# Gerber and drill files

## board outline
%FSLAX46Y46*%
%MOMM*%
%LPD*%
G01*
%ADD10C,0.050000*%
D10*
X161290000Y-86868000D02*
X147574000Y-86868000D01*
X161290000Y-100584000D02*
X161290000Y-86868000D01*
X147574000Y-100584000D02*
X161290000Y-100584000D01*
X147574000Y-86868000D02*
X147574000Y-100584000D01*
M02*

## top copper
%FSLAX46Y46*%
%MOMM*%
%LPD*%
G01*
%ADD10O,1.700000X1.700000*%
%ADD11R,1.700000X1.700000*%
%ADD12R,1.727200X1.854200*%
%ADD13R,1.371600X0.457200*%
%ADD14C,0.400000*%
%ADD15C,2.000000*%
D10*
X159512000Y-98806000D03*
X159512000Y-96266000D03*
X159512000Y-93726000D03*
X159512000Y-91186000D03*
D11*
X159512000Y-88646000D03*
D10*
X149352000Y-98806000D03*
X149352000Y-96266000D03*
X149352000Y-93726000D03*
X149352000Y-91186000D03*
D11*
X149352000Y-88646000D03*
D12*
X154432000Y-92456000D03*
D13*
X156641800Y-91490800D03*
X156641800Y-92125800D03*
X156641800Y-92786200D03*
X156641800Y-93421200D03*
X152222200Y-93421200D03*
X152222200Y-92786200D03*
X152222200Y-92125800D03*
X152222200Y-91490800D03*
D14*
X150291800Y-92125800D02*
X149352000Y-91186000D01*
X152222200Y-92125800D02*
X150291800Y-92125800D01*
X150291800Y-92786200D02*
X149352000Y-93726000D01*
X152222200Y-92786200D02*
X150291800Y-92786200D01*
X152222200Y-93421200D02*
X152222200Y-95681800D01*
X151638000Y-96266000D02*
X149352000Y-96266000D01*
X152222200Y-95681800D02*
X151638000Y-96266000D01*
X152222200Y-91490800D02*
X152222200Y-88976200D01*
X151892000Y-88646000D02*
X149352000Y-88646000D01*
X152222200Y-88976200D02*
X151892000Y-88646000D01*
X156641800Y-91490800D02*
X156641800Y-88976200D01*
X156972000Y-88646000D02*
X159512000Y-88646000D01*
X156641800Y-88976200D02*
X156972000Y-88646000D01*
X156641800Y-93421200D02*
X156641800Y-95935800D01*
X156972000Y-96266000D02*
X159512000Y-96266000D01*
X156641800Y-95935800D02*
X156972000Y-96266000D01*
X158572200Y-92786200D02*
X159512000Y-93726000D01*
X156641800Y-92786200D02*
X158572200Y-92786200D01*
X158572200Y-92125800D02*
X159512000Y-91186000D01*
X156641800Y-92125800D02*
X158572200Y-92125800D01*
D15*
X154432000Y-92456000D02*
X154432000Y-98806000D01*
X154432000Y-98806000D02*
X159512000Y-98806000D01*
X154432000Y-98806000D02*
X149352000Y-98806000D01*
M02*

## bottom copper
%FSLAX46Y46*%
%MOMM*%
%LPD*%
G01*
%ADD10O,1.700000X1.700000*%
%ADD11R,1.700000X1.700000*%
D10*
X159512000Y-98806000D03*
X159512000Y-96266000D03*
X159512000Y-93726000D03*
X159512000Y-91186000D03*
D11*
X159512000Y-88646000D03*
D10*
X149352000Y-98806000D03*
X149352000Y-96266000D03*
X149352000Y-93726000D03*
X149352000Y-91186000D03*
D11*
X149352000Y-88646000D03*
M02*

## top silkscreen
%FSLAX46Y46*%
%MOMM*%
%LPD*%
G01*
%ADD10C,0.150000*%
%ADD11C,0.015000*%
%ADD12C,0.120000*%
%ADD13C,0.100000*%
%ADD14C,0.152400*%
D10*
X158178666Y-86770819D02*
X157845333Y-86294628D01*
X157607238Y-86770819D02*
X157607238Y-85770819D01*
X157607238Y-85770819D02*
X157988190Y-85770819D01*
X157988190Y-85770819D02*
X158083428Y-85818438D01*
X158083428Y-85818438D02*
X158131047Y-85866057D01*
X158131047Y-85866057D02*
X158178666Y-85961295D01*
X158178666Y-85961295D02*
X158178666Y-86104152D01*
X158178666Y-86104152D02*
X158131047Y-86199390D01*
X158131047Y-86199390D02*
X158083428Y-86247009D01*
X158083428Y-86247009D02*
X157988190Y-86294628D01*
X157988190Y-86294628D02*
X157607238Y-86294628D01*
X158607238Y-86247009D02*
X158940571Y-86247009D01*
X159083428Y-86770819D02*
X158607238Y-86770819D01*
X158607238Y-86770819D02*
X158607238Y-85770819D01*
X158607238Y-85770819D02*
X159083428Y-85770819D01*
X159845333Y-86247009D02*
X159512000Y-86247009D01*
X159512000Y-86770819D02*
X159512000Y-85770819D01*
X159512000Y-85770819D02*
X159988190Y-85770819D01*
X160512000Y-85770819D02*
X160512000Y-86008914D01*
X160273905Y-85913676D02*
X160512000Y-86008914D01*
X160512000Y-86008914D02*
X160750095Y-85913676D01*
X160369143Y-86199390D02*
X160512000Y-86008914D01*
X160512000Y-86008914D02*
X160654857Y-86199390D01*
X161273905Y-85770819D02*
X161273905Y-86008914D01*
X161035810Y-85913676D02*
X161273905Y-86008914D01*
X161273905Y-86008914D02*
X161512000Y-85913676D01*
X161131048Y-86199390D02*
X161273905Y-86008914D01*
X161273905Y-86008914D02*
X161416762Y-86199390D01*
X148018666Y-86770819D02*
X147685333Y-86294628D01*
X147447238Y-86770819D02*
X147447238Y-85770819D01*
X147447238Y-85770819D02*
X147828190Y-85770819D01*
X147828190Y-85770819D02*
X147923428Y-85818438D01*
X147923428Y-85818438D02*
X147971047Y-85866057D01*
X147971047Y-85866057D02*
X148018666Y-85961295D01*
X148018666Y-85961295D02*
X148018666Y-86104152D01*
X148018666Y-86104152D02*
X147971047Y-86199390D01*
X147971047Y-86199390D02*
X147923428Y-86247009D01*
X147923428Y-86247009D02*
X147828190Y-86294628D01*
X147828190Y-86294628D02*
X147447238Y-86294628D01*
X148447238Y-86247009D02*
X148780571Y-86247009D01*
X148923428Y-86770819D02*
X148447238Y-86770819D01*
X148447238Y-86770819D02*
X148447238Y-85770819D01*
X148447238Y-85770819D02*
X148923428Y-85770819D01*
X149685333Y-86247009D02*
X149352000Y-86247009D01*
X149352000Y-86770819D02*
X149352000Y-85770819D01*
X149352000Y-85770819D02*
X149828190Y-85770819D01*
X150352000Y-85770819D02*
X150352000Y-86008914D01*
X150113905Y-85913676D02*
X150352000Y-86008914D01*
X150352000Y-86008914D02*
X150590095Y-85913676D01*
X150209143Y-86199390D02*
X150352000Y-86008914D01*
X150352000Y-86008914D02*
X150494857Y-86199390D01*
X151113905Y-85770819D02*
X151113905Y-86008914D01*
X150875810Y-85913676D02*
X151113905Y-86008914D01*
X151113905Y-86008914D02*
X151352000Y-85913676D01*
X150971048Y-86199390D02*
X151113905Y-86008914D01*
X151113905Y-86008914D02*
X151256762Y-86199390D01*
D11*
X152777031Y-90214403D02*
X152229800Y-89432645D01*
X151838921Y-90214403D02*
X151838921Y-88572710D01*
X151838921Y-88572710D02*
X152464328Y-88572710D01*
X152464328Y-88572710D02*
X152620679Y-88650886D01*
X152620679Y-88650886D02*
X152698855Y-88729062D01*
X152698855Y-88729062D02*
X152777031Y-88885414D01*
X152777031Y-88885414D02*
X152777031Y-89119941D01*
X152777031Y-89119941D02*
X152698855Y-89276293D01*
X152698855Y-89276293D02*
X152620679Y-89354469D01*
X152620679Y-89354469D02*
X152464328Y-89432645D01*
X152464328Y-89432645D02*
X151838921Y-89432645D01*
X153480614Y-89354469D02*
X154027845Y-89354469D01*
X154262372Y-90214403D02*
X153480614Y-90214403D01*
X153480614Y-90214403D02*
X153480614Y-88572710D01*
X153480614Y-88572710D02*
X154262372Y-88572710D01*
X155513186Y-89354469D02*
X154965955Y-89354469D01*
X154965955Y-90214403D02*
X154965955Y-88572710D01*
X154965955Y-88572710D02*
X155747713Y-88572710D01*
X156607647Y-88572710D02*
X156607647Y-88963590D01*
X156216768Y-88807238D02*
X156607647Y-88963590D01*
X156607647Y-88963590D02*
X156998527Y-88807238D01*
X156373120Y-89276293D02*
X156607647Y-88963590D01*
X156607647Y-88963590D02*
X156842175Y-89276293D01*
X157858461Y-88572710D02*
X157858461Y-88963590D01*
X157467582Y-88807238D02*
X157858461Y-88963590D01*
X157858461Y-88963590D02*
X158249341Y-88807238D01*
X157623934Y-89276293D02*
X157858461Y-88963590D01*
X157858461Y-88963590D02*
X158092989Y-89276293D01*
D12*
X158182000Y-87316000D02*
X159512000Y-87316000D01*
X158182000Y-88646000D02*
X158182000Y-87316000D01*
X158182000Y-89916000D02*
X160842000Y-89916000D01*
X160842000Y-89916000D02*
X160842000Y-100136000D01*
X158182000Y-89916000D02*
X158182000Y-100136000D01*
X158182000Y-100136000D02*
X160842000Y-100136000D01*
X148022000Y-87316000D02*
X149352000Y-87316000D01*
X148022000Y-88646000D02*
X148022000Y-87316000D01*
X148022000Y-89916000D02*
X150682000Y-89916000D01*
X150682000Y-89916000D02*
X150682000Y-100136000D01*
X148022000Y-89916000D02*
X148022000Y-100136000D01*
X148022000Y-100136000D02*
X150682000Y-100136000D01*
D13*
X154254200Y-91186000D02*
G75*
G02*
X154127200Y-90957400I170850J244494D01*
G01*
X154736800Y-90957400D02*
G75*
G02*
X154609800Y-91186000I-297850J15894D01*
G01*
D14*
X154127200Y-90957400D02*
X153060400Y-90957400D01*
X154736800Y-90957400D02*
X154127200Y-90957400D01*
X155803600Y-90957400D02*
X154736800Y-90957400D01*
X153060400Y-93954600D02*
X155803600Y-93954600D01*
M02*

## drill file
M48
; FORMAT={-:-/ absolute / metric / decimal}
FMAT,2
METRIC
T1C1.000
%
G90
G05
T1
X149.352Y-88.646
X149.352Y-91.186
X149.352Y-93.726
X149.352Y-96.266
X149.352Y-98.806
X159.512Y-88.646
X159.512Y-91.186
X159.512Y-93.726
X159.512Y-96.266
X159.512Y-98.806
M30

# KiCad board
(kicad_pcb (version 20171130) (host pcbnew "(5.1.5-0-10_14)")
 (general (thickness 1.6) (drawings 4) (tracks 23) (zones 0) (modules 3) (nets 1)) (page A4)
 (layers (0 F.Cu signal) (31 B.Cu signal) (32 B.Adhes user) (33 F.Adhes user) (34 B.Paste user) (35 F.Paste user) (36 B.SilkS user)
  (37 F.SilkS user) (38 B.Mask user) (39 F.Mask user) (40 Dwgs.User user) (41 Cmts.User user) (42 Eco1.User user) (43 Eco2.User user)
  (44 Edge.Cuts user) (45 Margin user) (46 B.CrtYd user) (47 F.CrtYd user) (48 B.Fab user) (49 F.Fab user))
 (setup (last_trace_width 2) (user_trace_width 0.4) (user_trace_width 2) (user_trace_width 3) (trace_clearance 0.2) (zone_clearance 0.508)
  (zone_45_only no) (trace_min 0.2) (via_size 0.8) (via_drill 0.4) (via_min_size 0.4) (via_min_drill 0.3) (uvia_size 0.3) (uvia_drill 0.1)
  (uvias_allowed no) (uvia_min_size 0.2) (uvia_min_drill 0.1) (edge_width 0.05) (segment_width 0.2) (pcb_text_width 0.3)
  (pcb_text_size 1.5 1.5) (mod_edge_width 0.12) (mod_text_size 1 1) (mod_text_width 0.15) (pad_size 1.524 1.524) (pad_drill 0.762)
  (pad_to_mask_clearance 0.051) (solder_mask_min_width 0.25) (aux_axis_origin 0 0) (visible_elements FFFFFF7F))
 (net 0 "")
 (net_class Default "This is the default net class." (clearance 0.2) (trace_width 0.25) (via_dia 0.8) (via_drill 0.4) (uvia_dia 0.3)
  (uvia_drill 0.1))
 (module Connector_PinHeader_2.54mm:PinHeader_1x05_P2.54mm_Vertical (layer F.Cu) (at 159.512 88.646)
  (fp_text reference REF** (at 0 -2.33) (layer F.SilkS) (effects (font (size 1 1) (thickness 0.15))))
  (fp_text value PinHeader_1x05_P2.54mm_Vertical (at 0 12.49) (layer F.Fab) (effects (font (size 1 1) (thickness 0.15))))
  (fp_line (start -1.33 -1.33) (end 0 -1.33) (layer F.SilkS) (width 0.12))
  (fp_line (start -1.33 0) (end -1.33 -1.33) (layer F.SilkS) (width 0.12))
  (fp_line (start -1.33 1.27) (end 1.33 1.27) (layer F.SilkS) (width 0.12))
  (fp_line (start 1.33 1.27) (end 1.33 11.49) (layer F.SilkS) (width 0.12))
  (fp_line (start -1.33 1.27) (end -1.33 11.49) (layer F.SilkS) (width 0.12))
  (fp_line (start -1.33 11.49) (end 1.33 11.49) (layer F.SilkS) (width 0.12))
  (pad 5 thru_hole oval (at 0 10.16) (size 1.7 1.7) (drill 1) (layers *.Cu *.Mask))
  (pad 4 thru_hole oval (at 0 7.62) (size 1.7 1.7) (drill 1) (layers *.Cu *.Mask))
  (pad 3 thru_hole oval (at 0 5.08) (size 1.7 1.7) (drill 1) (layers *.Cu *.Mask))
  (pad 2 thru_hole oval (at 0 2.54) (size 1.7 1.7) (drill 1) (layers *.Cu *.Mask))
  (pad 1 thru_hole rect (at 0 0) (size 1.7 1.7) (drill 1) (layers *.Cu *.Mask)))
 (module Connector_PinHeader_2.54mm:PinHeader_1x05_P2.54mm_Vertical (layer F.Cu) (at 149.352 88.646)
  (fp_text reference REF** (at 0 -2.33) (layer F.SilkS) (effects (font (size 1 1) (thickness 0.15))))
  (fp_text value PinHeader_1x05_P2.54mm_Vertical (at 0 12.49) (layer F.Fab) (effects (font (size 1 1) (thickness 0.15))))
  (fp_line (start -1.33 -1.33) (end 0 -1.33) (layer F.SilkS) (width 0.12))
  (fp_line (start -1.33 0) (end -1.33 -1.33) (layer F.SilkS) (width 0.12))
  (fp_line (start -1.33 1.27) (end 1.33 1.27) (layer F.SilkS) (width 0.12))
  (fp_line (start 1.33 1.27) (end 1.33 11.49) (layer F.SilkS) (width 0.12))
  (fp_line (start -1.33 1.27) (end -1.33 11.49) (layer F.SilkS) (width 0.12))
  (fp_line (start -1.33 11.49) (end 1.33 11.49) (layer F.SilkS) (width 0.12))
  (pad 5 thru_hole oval (at 0 10.16) (size 1.7 1.7) (drill 1) (layers *.Cu *.Mask))
  (pad 4 thru_hole oval (at 0 7.62) (size 1.7 1.7) (drill 1) (layers *.Cu *.Mask))
  (pad 3 thru_hole oval (at 0 5.08) (size 1.7 1.7) (drill 1) (layers *.Cu *.Mask))
  (pad 2 thru_hole oval (at 0 2.54) (size 1.7 1.7) (drill 1) (layers *.Cu *.Mask))
  (pad 1 thru_hole rect (at 0 0) (size 1.7 1.7) (drill 1) (layers *.Cu *.Mask)))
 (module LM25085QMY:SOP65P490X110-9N (layer F.Cu) (at 154.432 92.456)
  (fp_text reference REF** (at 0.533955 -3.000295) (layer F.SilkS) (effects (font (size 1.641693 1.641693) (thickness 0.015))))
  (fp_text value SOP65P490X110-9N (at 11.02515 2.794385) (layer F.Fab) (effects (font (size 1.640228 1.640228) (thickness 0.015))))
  (fp_arc (start -0.00695 -1.514494) (end -0.3048 -1.4986) (angle -52) (layer F.SilkS) (width 0.1))
  (fp_arc (start 0.00695 -1.514494) (end 0.1778 -1.27) (angle -52) (layer F.SilkS) (width 0.1))
  (fp_line (start -0.3048 -1.4986) (end -1.3716 -1.4986) (layer F.SilkS) (width 0.1524))
  (fp_line (start 0.3048 -1.4986) (end -0.3048 -1.4986) (layer F.SilkS) (width 0.1524))
  (fp_line (start 1.3716 -1.4986) (end 0.3048 -1.4986) (layer F.SilkS) (width 0.1524))
  (fp_line (start -1.3716 1.4986) (end 1.3716 1.4986) (layer F.SilkS) (width 0.1524))
  (pad 9 smd rect (at 0 0) (size 1.7272 1.8542) (layers F.Cu F.Paste F.Mask))
  (pad 8 smd rect (at 2.2098 -0.9652) (size 1.3716 0.4572) (layers F.Cu F.Paste F.Mask))
  (pad 7 smd rect (at 2.2098 -0.3302) (size 1.3716 0.4572) (layers F.Cu F.Paste F.Mask))
  (pad 6 smd rect (at 2.2098 0.3302) (size 1.3716 0.4572) (layers F.Cu F.Paste F.Mask))
  (pad 5 smd rect (at 2.2098 0.9652) (size 1.3716 0.4572) (layers F.Cu F.Paste F.Mask))
  (pad 4 smd rect (at -2.2098 0.9652) (size 1.3716 0.4572) (layers F.Cu F.Paste F.Mask))
  (pad 3 smd rect (at -2.2098 0.3302) (size 1.3716 0.4572) (layers F.Cu F.Paste F.Mask))
  (pad 2 smd rect (at -2.2098 -0.3302) (size 1.3716 0.4572) (layers F.Cu F.Paste F.Mask))
  (pad 1 smd rect (at -2.2098 -0.9652) (size 1.3716 0.4572) (layers F.Cu F.Paste F.Mask)))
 (gr_line (start 161.29 86.868) (end 147.574 86.868) (layer Edge.Cuts) (width 0.05))
 (gr_line (start 161.29 100.584) (end 161.29 86.868) (layer Edge.Cuts) (width 0.05))
 (gr_line (start 147.574 100.584) (end 161.29 100.584) (layer Edge.Cuts) (width 0.05))
 (gr_line (start 147.574 86.868) (end 147.574 100.584) (layer Edge.Cuts) (width 0.05))
 (segment (start 150.2918 92.1258) (end 149.352 91.186) (width 0.4) (layer F.Cu) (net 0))
 (segment (start 152.2222 92.1258) (end 150.2918 92.1258) (width 0.4) (layer F.Cu) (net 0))
 (segment (start 150.2918 92.7862) (end 149.352 93.726) (width 0.4) (layer F.Cu) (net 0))
 (segment (start 152.2222 92.7862) (end 150.2918 92.7862) (width 0.4) (layer F.Cu) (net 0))
 (segment (start 152.2222 93.4212) (end 152.2222 95.6818) (width 0.4) (layer F.Cu) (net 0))
 (segment (start 151.638 96.266) (end 149.352 96.266) (width 0.4) (layer F.Cu) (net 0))
 (segment (start 152.2222 95.6818) (end 151.638 96.266) (width 0.4) (layer F.Cu) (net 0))
 (segment (start 152.2222 91.4908) (end 152.2222 88.9762) (width 0.4) (layer F.Cu) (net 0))
 (segment (start 151.892 88.646) (end 149.352 88.646) (width 0.4) (layer F.Cu) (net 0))
 (segment (start 152.2222 88.9762) (end 151.892 88.646) (width 0.4) (layer F.Cu) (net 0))
 (segment (start 156.6418 91.4908) (end 156.6418 88.9762) (width 0.4) (layer F.Cu) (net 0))
 (segment (start 156.972 88.646) (end 159.512 88.646) (width 0.4) (layer F.Cu) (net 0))
 (segment (start 156.6418 88.9762) (end 156.972 88.646) (width 0.4) (layer F.Cu) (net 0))
 (segment (start 156.6418 93.4212) (end 156.6418 95.9358) (width 0.4) (layer F.Cu) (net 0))
 (segment (start 156.972 96.266) (end 159.512 96.266) (width 0.4) (layer F.Cu) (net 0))
 (segment (start 156.6418 95.9358) (end 156.972 96.266) (width 0.4) (layer F.Cu) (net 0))
 (segment (start 158.5722 92.7862) (end 159.512 93.726) (width 0.4) (layer F.Cu) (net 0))
 (segment (start 156.6418 92.7862) (end 158.5722 92.7862) (width 0.4) (layer F.Cu) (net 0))
 (segment (start 158.5722 92.1258) (end 159.512 91.186) (width 0.4) (layer F.Cu) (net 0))
 (segment (start 156.6418 92.1258) (end 158.5722 92.1258) (width 0.4) (layer F.Cu) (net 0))
 (segment (start 154.432 92.456) (end 154.432 98.806) (width 2) (layer F.Cu) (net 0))
 (segment (start 154.432 98.806) (end 159.512 98.806) (width 2) (layer F.Cu) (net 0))
 (segment (start 154.432 98.806) (end 149.352 98.806) (width 2) (layer F.Cu) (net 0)))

